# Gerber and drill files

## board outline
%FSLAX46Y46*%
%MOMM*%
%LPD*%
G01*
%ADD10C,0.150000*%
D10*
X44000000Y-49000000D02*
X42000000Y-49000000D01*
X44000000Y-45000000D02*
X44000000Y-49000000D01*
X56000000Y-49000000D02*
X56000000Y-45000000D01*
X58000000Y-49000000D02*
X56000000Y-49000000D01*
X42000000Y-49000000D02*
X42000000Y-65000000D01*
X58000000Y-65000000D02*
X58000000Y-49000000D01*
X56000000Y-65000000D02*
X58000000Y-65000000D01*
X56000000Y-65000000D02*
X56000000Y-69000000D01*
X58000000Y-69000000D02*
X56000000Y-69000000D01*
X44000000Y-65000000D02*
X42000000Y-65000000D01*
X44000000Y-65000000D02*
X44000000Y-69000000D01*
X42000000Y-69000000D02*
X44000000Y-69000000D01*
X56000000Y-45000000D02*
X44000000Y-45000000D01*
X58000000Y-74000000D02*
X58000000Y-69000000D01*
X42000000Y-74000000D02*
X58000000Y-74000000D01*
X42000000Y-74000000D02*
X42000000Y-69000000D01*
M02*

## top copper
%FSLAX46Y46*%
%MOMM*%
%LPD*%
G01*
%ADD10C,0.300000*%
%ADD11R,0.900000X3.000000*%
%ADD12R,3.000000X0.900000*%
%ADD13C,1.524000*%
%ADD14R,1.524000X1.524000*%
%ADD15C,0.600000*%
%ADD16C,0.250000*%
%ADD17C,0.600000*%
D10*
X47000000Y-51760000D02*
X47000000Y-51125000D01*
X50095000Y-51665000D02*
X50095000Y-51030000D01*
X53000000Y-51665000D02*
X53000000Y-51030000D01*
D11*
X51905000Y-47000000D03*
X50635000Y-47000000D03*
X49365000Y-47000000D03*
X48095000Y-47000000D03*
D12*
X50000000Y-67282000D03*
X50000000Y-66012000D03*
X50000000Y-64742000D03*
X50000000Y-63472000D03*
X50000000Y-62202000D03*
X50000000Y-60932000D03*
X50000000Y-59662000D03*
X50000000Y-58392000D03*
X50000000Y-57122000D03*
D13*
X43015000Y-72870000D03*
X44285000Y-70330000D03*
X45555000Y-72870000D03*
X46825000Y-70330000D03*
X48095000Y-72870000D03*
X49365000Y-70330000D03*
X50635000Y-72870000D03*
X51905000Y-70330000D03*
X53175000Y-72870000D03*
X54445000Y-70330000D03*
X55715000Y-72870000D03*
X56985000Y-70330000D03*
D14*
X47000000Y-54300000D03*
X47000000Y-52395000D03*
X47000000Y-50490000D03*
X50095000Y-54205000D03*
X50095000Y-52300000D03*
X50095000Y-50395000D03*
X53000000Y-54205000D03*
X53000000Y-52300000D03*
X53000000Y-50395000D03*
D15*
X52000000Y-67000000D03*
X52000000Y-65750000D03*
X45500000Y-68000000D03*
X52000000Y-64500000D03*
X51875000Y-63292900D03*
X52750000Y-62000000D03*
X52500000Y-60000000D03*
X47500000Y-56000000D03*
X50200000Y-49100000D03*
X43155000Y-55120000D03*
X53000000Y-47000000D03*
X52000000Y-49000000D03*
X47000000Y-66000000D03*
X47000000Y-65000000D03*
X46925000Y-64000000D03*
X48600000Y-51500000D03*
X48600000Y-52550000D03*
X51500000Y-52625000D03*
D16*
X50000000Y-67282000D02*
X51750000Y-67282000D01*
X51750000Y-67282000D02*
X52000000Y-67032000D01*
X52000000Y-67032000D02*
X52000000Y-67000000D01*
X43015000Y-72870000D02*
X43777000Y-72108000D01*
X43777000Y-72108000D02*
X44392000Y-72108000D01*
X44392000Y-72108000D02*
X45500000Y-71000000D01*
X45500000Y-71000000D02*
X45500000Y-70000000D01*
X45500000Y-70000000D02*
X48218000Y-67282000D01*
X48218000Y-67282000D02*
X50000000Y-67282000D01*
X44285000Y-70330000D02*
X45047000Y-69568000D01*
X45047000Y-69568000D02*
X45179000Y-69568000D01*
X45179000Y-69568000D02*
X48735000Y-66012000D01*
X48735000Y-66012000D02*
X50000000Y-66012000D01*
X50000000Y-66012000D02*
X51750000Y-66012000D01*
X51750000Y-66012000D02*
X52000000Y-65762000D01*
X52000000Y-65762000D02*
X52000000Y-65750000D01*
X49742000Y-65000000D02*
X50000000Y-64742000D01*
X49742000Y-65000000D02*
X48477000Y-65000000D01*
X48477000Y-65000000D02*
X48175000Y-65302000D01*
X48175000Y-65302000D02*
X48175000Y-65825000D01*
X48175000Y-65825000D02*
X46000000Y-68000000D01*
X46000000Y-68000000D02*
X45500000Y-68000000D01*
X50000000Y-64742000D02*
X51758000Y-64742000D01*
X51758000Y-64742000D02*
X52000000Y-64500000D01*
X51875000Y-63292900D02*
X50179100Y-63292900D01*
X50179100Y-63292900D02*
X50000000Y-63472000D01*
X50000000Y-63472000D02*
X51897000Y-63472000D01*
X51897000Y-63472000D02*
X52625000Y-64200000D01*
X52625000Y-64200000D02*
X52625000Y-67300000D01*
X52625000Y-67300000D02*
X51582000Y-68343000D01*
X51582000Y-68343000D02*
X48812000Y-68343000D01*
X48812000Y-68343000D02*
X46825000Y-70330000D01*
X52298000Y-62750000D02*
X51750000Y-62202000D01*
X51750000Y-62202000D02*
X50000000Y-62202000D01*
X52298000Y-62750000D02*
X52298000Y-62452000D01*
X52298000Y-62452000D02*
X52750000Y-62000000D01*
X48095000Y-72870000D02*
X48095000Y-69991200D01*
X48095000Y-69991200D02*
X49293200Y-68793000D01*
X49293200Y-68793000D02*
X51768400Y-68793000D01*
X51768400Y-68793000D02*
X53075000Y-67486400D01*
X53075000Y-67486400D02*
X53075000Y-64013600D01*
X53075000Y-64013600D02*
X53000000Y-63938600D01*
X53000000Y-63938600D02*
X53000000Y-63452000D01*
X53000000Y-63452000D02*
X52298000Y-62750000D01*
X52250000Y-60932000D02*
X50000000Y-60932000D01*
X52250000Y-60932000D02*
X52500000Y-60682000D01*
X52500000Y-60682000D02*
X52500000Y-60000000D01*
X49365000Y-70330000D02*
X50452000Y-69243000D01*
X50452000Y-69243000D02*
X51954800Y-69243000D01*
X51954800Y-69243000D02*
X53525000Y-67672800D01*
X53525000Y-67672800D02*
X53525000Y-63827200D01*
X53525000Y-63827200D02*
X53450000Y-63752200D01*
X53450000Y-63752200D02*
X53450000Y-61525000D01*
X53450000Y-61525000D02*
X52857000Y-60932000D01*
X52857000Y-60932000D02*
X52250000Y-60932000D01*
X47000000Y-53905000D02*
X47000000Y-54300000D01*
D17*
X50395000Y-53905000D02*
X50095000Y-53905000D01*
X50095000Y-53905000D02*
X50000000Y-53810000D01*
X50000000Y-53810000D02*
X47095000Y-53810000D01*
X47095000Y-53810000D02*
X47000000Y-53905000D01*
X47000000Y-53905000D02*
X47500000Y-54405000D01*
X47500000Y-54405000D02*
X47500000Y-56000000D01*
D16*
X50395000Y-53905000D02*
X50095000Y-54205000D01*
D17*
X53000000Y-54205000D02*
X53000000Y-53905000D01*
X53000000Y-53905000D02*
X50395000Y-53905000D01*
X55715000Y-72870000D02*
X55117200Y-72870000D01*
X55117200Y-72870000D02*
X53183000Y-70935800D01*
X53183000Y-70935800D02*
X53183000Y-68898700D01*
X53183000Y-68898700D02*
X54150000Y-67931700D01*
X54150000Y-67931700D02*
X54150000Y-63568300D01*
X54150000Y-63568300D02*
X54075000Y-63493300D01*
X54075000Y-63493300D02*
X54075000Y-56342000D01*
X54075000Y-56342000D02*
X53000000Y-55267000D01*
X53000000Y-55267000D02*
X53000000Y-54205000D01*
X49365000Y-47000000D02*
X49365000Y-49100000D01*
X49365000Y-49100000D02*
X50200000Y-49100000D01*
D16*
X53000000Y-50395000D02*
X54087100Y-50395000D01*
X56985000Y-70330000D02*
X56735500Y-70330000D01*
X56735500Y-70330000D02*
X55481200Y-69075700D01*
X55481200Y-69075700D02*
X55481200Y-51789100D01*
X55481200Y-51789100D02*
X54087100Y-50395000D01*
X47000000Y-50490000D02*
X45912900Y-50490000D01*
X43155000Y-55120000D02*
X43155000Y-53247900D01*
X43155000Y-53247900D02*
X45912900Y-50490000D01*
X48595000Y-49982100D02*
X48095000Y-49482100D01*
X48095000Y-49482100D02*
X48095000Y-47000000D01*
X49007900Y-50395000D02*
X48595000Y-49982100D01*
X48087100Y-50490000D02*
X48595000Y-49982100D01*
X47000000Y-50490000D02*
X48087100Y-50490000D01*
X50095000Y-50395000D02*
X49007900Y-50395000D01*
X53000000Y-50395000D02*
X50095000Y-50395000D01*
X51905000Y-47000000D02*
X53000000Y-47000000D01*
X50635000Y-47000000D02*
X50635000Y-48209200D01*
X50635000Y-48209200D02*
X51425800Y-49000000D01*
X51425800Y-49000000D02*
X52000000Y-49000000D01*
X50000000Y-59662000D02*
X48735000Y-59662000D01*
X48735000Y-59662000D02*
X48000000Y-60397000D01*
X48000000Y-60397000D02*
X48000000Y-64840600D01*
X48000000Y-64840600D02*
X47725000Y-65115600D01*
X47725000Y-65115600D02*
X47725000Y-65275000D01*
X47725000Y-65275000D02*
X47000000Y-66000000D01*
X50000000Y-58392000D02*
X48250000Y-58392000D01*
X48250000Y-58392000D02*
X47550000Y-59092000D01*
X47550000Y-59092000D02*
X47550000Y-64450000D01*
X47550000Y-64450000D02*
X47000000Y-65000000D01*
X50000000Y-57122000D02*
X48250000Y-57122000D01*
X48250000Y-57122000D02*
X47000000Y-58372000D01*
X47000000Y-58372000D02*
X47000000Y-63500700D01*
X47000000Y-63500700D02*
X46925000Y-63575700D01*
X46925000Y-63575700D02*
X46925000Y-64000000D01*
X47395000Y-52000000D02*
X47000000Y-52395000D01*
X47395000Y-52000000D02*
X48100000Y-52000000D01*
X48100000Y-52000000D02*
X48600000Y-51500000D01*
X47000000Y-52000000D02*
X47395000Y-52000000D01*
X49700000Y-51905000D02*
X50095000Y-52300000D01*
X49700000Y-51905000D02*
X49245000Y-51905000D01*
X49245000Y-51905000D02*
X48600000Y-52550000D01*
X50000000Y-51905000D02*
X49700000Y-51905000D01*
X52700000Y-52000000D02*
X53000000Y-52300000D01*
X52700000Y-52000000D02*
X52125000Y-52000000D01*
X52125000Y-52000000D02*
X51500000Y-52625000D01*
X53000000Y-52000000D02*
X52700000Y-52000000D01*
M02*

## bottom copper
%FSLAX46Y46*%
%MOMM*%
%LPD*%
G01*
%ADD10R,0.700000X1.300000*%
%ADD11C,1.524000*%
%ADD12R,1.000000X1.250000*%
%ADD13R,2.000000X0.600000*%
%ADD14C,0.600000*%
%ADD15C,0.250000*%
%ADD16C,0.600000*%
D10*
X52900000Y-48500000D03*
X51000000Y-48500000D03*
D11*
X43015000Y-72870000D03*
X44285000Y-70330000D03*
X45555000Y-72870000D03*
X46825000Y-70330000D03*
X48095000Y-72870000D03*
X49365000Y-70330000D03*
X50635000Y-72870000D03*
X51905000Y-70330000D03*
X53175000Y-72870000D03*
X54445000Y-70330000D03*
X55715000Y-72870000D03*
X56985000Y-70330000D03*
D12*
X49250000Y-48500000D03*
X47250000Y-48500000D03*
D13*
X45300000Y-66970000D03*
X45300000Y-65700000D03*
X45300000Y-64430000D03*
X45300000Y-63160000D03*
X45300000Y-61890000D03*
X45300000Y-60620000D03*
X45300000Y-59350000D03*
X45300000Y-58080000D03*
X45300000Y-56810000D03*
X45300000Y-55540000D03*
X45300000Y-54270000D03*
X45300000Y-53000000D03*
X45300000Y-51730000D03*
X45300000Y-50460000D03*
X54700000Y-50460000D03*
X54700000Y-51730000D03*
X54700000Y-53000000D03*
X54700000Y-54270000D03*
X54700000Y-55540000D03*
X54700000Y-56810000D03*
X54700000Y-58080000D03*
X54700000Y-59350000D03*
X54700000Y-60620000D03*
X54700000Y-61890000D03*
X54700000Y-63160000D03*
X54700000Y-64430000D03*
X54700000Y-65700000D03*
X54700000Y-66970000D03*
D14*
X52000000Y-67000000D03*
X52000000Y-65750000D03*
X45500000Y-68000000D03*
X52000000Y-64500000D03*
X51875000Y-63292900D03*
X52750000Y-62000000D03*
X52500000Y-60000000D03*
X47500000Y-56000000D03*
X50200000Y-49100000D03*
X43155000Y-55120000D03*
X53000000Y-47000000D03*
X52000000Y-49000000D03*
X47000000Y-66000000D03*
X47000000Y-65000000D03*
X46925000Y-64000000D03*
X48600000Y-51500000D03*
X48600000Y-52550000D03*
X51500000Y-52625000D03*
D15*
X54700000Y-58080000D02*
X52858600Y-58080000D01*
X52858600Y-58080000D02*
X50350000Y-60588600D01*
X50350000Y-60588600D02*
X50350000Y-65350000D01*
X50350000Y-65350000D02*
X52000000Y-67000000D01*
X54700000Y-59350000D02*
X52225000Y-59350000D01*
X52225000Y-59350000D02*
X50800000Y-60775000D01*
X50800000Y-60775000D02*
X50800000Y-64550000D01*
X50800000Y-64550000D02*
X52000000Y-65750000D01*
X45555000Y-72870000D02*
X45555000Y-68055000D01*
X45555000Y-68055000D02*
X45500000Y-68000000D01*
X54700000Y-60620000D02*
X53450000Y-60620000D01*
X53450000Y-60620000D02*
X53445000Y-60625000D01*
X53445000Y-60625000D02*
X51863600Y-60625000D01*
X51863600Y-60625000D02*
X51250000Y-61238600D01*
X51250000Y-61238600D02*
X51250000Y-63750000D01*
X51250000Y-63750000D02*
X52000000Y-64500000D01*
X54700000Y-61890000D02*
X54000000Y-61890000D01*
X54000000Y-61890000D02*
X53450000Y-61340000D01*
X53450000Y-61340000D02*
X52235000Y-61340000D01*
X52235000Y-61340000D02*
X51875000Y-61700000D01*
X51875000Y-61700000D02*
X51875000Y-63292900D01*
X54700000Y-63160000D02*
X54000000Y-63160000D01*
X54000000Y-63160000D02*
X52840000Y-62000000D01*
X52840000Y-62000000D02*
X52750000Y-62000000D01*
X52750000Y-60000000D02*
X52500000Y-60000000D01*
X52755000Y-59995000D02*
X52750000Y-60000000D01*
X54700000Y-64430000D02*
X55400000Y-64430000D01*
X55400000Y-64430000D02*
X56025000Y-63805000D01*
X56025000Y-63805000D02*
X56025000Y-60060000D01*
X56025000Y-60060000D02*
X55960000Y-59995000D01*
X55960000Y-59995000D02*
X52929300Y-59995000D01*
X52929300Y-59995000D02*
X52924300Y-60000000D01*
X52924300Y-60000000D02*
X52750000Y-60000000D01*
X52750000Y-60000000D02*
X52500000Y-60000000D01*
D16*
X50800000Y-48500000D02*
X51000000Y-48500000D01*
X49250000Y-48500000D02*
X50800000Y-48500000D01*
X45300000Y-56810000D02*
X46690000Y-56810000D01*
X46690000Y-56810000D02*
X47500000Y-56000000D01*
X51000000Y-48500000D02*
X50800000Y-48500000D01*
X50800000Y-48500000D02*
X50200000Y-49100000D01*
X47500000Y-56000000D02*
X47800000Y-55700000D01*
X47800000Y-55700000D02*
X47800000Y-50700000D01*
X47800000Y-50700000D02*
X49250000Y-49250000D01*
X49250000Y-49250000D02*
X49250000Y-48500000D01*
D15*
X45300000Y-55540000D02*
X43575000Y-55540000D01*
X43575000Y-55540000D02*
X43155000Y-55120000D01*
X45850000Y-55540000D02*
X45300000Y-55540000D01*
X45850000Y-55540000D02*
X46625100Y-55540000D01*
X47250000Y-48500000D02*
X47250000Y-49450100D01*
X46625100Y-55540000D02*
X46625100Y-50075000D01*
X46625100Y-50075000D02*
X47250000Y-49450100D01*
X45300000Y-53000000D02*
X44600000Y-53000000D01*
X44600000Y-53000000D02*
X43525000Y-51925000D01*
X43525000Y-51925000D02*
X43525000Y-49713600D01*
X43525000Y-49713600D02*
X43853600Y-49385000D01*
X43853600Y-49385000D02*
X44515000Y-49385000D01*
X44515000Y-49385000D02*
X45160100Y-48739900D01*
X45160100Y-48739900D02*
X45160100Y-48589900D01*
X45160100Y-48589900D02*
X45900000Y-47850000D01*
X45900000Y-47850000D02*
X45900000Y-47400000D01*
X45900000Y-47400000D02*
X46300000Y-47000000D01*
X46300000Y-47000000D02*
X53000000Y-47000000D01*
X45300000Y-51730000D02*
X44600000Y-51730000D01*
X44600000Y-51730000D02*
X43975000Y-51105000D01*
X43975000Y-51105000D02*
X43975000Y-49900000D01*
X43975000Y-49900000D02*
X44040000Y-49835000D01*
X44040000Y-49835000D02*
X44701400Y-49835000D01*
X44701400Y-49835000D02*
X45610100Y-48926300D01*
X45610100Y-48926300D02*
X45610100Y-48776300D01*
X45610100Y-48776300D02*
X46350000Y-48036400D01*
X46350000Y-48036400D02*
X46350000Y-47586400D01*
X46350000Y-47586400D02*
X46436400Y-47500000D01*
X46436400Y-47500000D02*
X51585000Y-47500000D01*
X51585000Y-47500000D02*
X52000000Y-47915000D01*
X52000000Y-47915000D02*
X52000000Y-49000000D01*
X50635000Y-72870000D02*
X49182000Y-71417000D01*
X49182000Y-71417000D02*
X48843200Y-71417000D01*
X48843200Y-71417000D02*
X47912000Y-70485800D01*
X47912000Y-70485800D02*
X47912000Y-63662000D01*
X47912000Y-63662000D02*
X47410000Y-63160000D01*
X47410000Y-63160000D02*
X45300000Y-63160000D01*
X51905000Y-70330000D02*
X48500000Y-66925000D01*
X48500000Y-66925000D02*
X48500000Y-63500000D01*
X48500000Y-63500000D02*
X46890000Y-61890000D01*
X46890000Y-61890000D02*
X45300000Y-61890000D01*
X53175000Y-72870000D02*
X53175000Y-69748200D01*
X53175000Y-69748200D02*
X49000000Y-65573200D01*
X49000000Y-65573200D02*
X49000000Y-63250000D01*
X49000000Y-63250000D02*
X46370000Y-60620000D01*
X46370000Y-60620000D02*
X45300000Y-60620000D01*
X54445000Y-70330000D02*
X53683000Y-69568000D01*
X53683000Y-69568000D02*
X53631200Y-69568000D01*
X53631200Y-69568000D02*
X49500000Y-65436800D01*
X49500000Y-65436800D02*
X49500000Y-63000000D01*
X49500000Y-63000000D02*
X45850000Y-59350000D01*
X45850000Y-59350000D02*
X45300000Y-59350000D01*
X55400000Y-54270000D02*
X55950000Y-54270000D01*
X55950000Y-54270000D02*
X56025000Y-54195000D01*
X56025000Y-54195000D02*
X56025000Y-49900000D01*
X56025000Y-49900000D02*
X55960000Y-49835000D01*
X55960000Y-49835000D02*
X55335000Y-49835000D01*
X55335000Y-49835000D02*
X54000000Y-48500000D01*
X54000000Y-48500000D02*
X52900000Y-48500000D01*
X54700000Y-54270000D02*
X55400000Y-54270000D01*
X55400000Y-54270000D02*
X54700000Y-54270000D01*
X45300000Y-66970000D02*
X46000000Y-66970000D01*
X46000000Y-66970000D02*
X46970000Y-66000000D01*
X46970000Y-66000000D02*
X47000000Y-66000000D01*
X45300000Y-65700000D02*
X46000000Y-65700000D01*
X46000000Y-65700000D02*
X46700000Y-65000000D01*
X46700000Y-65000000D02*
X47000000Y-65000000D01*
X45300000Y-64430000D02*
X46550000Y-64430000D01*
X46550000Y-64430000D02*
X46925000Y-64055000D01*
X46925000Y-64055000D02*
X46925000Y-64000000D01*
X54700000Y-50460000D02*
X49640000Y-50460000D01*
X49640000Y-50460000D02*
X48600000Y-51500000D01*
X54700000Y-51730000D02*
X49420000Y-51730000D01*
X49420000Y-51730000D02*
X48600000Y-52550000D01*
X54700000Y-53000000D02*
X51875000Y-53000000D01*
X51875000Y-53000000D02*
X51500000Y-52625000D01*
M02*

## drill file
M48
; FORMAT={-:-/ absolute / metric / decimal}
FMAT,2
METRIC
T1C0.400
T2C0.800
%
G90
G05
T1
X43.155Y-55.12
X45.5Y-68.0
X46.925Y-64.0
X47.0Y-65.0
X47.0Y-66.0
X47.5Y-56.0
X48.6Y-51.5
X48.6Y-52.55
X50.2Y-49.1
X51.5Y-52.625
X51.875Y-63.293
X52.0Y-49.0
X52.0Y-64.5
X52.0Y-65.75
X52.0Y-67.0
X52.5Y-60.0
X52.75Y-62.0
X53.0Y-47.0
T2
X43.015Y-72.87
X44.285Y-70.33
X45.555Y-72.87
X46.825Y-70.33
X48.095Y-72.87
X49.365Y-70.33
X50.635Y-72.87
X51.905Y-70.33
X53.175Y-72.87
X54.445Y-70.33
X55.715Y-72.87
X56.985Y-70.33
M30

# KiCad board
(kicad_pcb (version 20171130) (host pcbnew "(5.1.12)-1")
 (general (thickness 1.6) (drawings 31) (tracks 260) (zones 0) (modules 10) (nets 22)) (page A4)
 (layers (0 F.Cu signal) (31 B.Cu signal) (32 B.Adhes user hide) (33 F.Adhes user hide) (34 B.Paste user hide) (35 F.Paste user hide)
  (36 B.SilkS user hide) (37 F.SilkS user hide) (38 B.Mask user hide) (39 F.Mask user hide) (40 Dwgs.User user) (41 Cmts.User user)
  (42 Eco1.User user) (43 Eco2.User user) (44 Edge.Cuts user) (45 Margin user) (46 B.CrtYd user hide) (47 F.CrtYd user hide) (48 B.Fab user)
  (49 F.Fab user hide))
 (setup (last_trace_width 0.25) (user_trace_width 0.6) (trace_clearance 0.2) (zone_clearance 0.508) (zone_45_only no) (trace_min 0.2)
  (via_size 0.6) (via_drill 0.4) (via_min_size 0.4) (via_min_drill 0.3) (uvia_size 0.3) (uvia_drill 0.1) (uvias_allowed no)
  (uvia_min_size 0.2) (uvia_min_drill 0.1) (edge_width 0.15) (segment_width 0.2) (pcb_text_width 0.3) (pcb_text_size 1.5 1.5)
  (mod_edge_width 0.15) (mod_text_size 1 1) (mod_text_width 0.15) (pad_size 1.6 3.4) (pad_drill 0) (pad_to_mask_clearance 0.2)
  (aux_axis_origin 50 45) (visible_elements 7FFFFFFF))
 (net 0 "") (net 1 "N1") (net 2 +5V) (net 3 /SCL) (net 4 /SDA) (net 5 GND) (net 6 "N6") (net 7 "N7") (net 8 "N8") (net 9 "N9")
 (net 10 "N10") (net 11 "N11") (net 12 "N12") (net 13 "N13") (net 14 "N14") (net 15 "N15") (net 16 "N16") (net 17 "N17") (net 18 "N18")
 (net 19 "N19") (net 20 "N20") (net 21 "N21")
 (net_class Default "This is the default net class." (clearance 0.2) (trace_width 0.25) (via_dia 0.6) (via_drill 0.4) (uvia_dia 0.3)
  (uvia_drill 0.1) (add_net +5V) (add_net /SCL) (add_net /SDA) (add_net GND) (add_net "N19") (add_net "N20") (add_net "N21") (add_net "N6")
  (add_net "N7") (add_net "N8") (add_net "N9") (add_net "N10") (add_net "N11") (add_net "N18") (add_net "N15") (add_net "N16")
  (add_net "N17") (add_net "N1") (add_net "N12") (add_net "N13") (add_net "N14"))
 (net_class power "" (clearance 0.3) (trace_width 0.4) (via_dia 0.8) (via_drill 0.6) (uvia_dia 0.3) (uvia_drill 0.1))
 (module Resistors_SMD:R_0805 (layer B.Cu) (at 51.95 48.5 180)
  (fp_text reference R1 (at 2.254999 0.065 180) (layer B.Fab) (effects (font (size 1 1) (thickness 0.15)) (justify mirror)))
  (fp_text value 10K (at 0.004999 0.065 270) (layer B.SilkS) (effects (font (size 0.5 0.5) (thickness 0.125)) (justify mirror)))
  (pad 1 smd rect (at -0.95 0 180) (size 0.7 1.3) (layers B.Cu B.Paste B.Mask) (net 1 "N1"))
  (pad 2 smd rect (at 0.95 0 180) (size 0.7 1.3) (layers B.Cu B.Paste B.Mask) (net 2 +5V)))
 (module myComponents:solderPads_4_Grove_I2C (layer F.Cu) (at 50 47 180)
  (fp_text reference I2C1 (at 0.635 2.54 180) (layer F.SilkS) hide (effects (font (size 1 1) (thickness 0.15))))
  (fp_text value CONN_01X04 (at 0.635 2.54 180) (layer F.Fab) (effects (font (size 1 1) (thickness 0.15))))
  (pad 1 smd rect (at -1.905 0 180) (size 0.9 3) (layers F.Cu F.Paste F.Mask) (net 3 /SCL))
  (pad 2 smd rect (at -0.635 0 180) (size 0.9 3) (layers F.Cu F.Paste F.Mask) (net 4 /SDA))
  (pad 3 smd rect (at 0.635 0 180) (size 0.9 3) (layers F.Cu F.Paste F.Mask) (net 2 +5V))
  (pad 4 smd rect (at 1.905 0 180) (size 0.9 3) (layers F.Cu F.Paste F.Mask) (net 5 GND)))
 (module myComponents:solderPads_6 (layer F.Cu) (at 50 64.107 90)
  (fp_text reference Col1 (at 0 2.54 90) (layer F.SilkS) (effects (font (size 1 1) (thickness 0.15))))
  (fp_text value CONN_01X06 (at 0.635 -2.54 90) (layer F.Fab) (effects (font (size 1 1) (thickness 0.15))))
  (pad 1 smd rect (at -3.175 0 90) (size 0.9 3) (layers F.Cu F.Paste F.Mask) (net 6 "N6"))
  (pad 2 smd rect (at -1.905 0 90) (size 0.9 3) (layers F.Cu F.Paste F.Mask) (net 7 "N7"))
  (pad 3 smd rect (at -0.635 0 90) (size 0.9 3) (layers F.Cu F.Paste F.Mask) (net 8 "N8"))
  (pad 4 smd rect (at 0.635 0 90) (size 0.9 3) (layers F.Cu F.Paste F.Mask) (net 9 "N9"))
  (pad 5 smd rect (at 1.905 0 90) (size 0.9 3) (layers F.Cu F.Paste F.Mask) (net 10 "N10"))
  (pad 6 smd rect (at 3.175 0 90) (size 0.9 3) (layers F.Cu F.Paste F.Mask) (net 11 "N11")))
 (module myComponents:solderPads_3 (layer F.Cu) (at 50 58.392 90)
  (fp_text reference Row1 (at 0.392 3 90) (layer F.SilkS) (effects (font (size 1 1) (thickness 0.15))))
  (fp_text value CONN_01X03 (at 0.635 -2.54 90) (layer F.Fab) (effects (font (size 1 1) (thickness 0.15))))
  (pad 1 smd rect (at -1.27 0 90) (size 0.9 3) (layers F.Cu F.Paste F.Mask) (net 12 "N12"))
  (pad 2 smd rect (at 0 0 90) (size 0.9 3) (layers F.Cu F.Paste F.Mask) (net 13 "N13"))
  (pad 3 smd rect (at 1.27 0 90) (size 0.9 3) (layers F.Cu F.Paste F.Mask) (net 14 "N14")))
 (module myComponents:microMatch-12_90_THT (layer F.Cu) (at 50 71.6)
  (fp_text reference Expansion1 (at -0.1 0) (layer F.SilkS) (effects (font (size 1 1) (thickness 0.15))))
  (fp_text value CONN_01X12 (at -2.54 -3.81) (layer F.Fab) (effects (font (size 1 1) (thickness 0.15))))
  (pad 1 thru_hole circle (at -6.985 1.27) (size 1.524 1.524) (drill 0.8) (layers *.Cu *.Mask) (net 6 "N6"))
  (pad 2 thru_hole circle (at -5.715 -1.27) (size 1.524 1.524) (drill 0.8) (layers *.Cu *.Mask) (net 7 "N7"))
  (pad 3 thru_hole circle (at -4.445 1.27) (size 1.524 1.524) (drill 0.8) (layers *.Cu *.Mask) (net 8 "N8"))
  (pad 4 thru_hole circle (at -3.175 -1.27) (size 1.524 1.524) (drill 0.8) (layers *.Cu *.Mask) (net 9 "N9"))
  (pad 5 thru_hole circle (at -1.905 1.27) (size 1.524 1.524) (drill 0.8) (layers *.Cu *.Mask) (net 10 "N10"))
  (pad 6 thru_hole circle (at -0.635 -1.27) (size 1.524 1.524) (drill 0.8) (layers *.Cu *.Mask) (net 11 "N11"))
  (pad 7 thru_hole circle (at 0.635 1.27) (size 1.524 1.524) (drill 0.8) (layers *.Cu *.Mask) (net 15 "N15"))
  (pad 8 thru_hole circle (at 1.905 -1.27) (size 1.524 1.524) (drill 0.8) (layers *.Cu *.Mask) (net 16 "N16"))
  (pad 9 thru_hole circle (at 3.175 1.27) (size 1.524 1.524) (drill 0.8) (layers *.Cu *.Mask) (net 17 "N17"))
  (pad 10 thru_hole circle (at 4.445 -1.27) (size 1.524 1.524) (drill 0.8) (layers *.Cu *.Mask) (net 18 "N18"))
  (pad 11 thru_hole circle (at 5.715 1.27) (size 1.524 1.524) (drill 0.8) (layers *.Cu *.Mask) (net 2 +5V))
  (pad 12 thru_hole circle (at 6.985 -1.27) (size 1.524 1.524) (drill 0.8) (layers *.Cu *.Mask) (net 5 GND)))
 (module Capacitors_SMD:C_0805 (layer B.Cu) (at 48.25 48.5 180)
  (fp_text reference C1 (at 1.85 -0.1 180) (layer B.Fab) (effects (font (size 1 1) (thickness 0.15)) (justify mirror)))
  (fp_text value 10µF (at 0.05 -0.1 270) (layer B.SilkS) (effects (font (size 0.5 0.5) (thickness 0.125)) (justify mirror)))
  (pad 1 smd rect (at -1 0 180) (size 1 1.25) (layers B.Cu B.Paste B.Mask) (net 2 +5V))
  (pad 2 smd rect (at 1 0 180) (size 1 1.25) (layers B.Cu B.Paste B.Mask) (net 5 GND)))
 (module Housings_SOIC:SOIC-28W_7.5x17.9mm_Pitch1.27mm (layer B.Cu) (at 50 58.715)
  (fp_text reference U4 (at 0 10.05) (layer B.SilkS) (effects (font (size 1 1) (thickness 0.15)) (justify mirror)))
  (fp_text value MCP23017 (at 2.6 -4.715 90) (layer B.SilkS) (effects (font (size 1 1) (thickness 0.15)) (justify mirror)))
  (pad 1 smd rect (at -4.7 8.255) (size 2 0.6) (layers B.Cu B.Paste B.Mask) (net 12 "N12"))
  (pad 2 smd rect (at -4.7 6.985) (size 2 0.6) (layers B.Cu B.Paste B.Mask) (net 13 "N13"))
  (pad 3 smd rect (at -4.7 5.715) (size 2 0.6) (layers B.Cu B.Paste B.Mask) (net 14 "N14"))
  (pad 4 smd rect (at -4.7 4.445) (size 2 0.6) (layers B.Cu B.Paste B.Mask) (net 15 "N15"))
  (pad 5 smd rect (at -4.7 3.175) (size 2 0.6) (layers B.Cu B.Paste B.Mask) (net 16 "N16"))
  (pad 6 smd rect (at -4.7 1.905) (size 2 0.6) (layers B.Cu B.Paste B.Mask) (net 17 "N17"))
  (pad 7 smd rect (at -4.7 0.635) (size 2 0.6) (layers B.Cu B.Paste B.Mask) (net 18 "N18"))
  (pad 8 smd rect (at -4.7 -0.635) (size 2 0.6) (layers B.Cu B.Paste B.Mask))
  (pad 9 smd rect (at -4.7 -1.905) (size 2 0.6) (layers B.Cu B.Paste B.Mask) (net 2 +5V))
  (pad 10 smd rect (at -4.7 -3.175) (size 2 0.6) (layers B.Cu B.Paste B.Mask) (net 5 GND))
  (pad 11 smd rect (at -4.7 -4.445) (size 2 0.6) (layers B.Cu B.Paste B.Mask))
  (pad 12 smd rect (at -4.7 -5.715) (size 2 0.6) (layers B.Cu B.Paste B.Mask) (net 3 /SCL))
  (pad 13 smd rect (at -4.7 -6.985) (size 2 0.6) (layers B.Cu B.Paste B.Mask) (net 4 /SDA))
  (pad 14 smd rect (at -4.7 -8.255) (size 2 0.6) (layers B.Cu B.Paste B.Mask))
  (pad 15 smd rect (at 4.7 -8.255) (size 2 0.6) (layers B.Cu B.Paste B.Mask) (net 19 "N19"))
  (pad 16 smd rect (at 4.7 -6.985) (size 2 0.6) (layers B.Cu B.Paste B.Mask) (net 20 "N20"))
  (pad 17 smd rect (at 4.7 -5.715) (size 2 0.6) (layers B.Cu B.Paste B.Mask) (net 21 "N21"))
  (pad 18 smd rect (at 4.7 -4.445) (size 2 0.6) (layers B.Cu B.Paste B.Mask) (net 1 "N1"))
  (pad 19 smd rect (at 4.7 -3.175) (size 2 0.6) (layers B.Cu B.Paste B.Mask))
  (pad 20 smd rect (at 4.7 -1.905) (size 2 0.6) (layers B.Cu B.Paste B.Mask))
  (pad 21 smd rect (at 4.7 -0.635) (size 2 0.6) (layers B.Cu B.Paste B.Mask) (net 6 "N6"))
  (pad 22 smd rect (at 4.7 0.635) (size 2 0.6) (layers B.Cu B.Paste B.Mask) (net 7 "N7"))
  (pad 23 smd rect (at 4.7 1.905) (size 2 0.6) (layers B.Cu B.Paste B.Mask) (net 8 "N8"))
  (pad 24 smd rect (at 4.7 3.175) (size 2 0.6) (layers B.Cu B.Paste B.Mask) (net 9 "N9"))
  (pad 25 smd rect (at 4.7 4.445) (size 2 0.6) (layers B.Cu B.Paste B.Mask) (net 10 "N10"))
  (pad 26 smd rect (at 4.7 5.715) (size 2 0.6) (layers B.Cu B.Paste B.Mask) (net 11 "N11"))
  (pad 27 smd rect (at 4.7 6.985) (size 2 0.6) (layers B.Cu B.Paste B.Mask))
  (pad 28 smd rect (at 4.7 8.255) (size 2 0.6) (layers B.Cu B.Paste B.Mask)))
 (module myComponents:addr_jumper (layer F.Cu) (at 47 52.395 90)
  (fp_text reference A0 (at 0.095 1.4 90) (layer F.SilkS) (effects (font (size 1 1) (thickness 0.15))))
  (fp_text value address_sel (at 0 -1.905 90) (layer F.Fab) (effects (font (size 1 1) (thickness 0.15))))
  (fp_line (start 0.635 0) (end 1.27 0) (layer F.Cu) (width 0.3))
  (pad 1 smd rect (at -1.905 0 90) (size 1.524 1.524) (layers F.Cu F.Paste F.Mask) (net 2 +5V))
  (pad 2 smd rect (at 0 0 90) (size 1.524 1.524) (layers F.Cu F.Paste F.Mask) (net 19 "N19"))
  (pad 3 smd rect (at 1.905 0 90) (size 1.524 1.524) (layers F.Cu F.Paste F.Mask) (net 5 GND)))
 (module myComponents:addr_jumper (layer F.Cu) (at 50.095 52.3 90)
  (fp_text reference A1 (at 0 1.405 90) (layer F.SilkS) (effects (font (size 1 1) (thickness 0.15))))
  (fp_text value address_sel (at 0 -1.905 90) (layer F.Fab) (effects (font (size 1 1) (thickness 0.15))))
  (fp_line (start 0.635 0) (end 1.27 0) (layer F.Cu) (width 0.3))
  (pad 1 smd rect (at -1.905 0 90) (size 1.524 1.524) (layers F.Cu F.Paste F.Mask) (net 2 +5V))
  (pad 2 smd rect (at 0 0 90) (size 1.524 1.524) (layers F.Cu F.Paste F.Mask) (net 20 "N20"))
  (pad 3 smd rect (at 1.905 0 90) (size 1.524 1.524) (layers F.Cu F.Paste F.Mask) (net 5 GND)))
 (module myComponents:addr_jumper (layer F.Cu) (at 53 52.3 90)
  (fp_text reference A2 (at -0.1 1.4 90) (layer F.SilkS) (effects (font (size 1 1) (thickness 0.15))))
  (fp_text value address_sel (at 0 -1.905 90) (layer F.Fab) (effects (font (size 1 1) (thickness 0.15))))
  (fp_line (start 0.635 0) (end 1.27 0) (layer F.Cu) (width 0.3))
  (pad 1 smd rect (at -1.905 0 90) (size 1.524 1.524) (layers F.Cu F.Paste F.Mask) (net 2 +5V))
  (pad 2 smd rect (at 0 0 90) (size 1.524 1.524) (layers F.Cu F.Paste F.Mask) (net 21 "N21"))
  (pad 3 smd rect (at 1.905 0 90) (size 1.524 1.524) (layers F.Cu F.Paste F.Mask) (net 5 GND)))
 (gr_line (start 44 49) (end 42 49) (layer Edge.Cuts) (width 0.15))
 (gr_line (start 44 45) (end 44 49) (layer Edge.Cuts) (width 0.15))
 (gr_line (start 56 49) (end 56 45) (layer Edge.Cuts) (width 0.15))
 (gr_line (start 58 49) (end 56 49) (layer Edge.Cuts) (width 0.15))
 (gr_line (start 42 49) (end 42 65) (layer Edge.Cuts) (width 0.15))
 (gr_line (start 58 65) (end 58 49) (layer Edge.Cuts) (width 0.15))
 (gr_line (start 56 65) (end 58 65) (layer Edge.Cuts) (width 0.15))
 (gr_line (start 56 65) (end 56 69) (layer Edge.Cuts) (width 0.15))
 (gr_line (start 58 69) (end 56 69) (layer Edge.Cuts) (width 0.15))
 (gr_line (start 44 65) (end 42 65) (layer Edge.Cuts) (width 0.15))
 (gr_line (start 44 65) (end 44 69) (layer Edge.Cuts) (width 0.15))
 (gr_line (start 42 69) (end 44 69) (layer Edge.Cuts) (width 0.15))
 (gr_line (start 56 45) (end 44 45) (layer Edge.Cuts) (width 0.15))
 (gr_line (start 58 74) (end 58 69) (layer Edge.Cuts) (width 0.15))
 (gr_line (start 42 74) (end 58 74) (layer Edge.Cuts) (width 0.15))
 (gr_line (start 42 74) (end 42 69) (layer Edge.Cuts) (width 0.15))
 (segment (start 50 67.282) (end 51.75 67.282) (width 0.25) (layer F.Cu) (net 6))
 (segment (start 51.75 67.282) (end 52 67.032) (width 0.25) (layer F.Cu) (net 6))
 (segment (start 52 67.032) (end 52 67) (width 0.25) (layer F.Cu) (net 6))
 (segment (start 54.7 58.08) (end 52.8586 58.08) (width 0.25) (layer B.Cu) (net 6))
 (segment (start 52.8586 58.08) (end 50.35 60.5886) (width 0.25) (layer B.Cu) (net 6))
 (segment (start 50.35 60.5886) (end 50.35 65.35) (width 0.25) (layer B.Cu) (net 6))
 (segment (start 50.35 65.35) (end 52 67) (width 0.25) (layer B.Cu) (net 6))
 (segment (start 43.015 72.87) (end 43.777 72.108) (width 0.25) (layer F.Cu) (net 6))
 (segment (start 43.777 72.108) (end 44.392 72.108) (width 0.25) (layer F.Cu) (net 6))
 (segment (start 44.392 72.108) (end 45.5 71) (width 0.25) (layer F.Cu) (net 6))
 (segment (start 45.5 71) (end 45.5 70) (width 0.25) (layer F.Cu) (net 6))
 (segment (start 45.5 70) (end 48.218 67.282) (width 0.25) (layer F.Cu) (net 6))
 (segment (start 48.218 67.282) (end 50 67.282) (width 0.25) (layer F.Cu) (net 6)) (via (at 52 67) (size 0.6) (layers F.Cu B.Cu) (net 6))
 (segment (start 44.285 70.33) (end 45.047 69.568) (width 0.25) (layer F.Cu) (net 7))
 (segment (start 45.047 69.568) (end 45.179 69.568) (width 0.25) (layer F.Cu) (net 7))
 (segment (start 45.179 69.568) (end 48.735 66.012) (width 0.25) (layer F.Cu) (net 7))
 (segment (start 48.735 66.012) (end 50 66.012) (width 0.25) (layer F.Cu) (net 7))
 (segment (start 54.7 59.35) (end 52.225 59.35) (width 0.25) (layer B.Cu) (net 7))
 (segment (start 52.225 59.35) (end 50.8 60.775) (width 0.25) (layer B.Cu) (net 7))
 (segment (start 50.8 60.775) (end 50.8 64.55) (width 0.25) (layer B.Cu) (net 7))
 (segment (start 50.8 64.55) (end 52 65.75) (width 0.25) (layer B.Cu) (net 7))
 (segment (start 50 66.012) (end 51.75 66.012) (width 0.25) (layer F.Cu) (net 7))
 (segment (start 51.75 66.012) (end 52 65.762) (width 0.25) (layer F.Cu) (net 7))
 (segment (start 52 65.762) (end 52 65.75) (width 0.25) (layer F.Cu) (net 7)) (via (at 52 65.75) (size 0.6) (layers F.Cu B.Cu) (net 7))
 (segment (start 49.742 65) (end 50 64.742) (width 0.25) (layer F.Cu) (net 8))
 (segment (start 49.742 65) (end 48.477 65) (width 0.25) (layer F.Cu) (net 8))
 (segment (start 48.477 65) (end 48.175 65.302) (width 0.25) (layer F.Cu) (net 8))
 (segment (start 48.175 65.302) (end 48.175 65.825) (width 0.25) (layer F.Cu) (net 8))
 (segment (start 48.175 65.825) (end 46 68) (width 0.25) (layer F.Cu) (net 8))
 (segment (start 46 68) (end 45.5 68) (width 0.25) (layer F.Cu) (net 8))
 (segment (start 45.555 72.87) (end 45.555 68.055) (width 0.25) (layer B.Cu) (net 8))
 (segment (start 45.555 68.055) (end 45.5 68) (width 0.25) (layer B.Cu) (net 8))
 (segment (start 54.7 60.62) (end 53.45 60.62) (width 0.25) (layer B.Cu) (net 8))
 (segment (start 53.45 60.62) (end 53.445 60.625) (width 0.25) (layer B.Cu) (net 8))
 (segment (start 53.445 60.625) (end 51.8636 60.625) (width 0.25) (layer B.Cu) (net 8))
 (segment (start 51.8636 60.625) (end 51.25 61.2386) (width 0.25) (layer B.Cu) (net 8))
 (segment (start 51.25 61.2386) (end 51.25 63.75) (width 0.25) (layer B.Cu) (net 8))
 (segment (start 51.25 63.75) (end 52 64.5) (width 0.25) (layer B.Cu) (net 8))
 (segment (start 50 64.742) (end 51.758 64.742) (width 0.25) (layer F.Cu) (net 8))
 (segment (start 51.758 64.742) (end 52 64.5) (width 0.25) (layer F.Cu) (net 8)) (via (at 45.5 68) (size 0.6) (layers F.Cu B.Cu) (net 8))
 (via (at 52 64.5) (size 0.6) (layers F.Cu B.Cu) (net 8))
 (segment (start 51.875 63.2929) (end 50.1791 63.2929) (width 0.25) (layer F.Cu) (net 9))
 (segment (start 50.1791 63.2929) (end 50 63.472) (width 0.25) (layer F.Cu) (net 9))
 (segment (start 54.7 61.89) (end 54 61.89) (width 0.25) (layer B.Cu) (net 9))
 (segment (start 54 61.89) (end 53.45 61.34) (width 0.25) (layer B.Cu) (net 9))
 (segment (start 53.45 61.34) (end 52.235 61.34) (width 0.25) (layer B.Cu) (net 9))
 (segment (start 52.235 61.34) (end 51.875 61.7) (width 0.25) (layer B.Cu) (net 9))
 (segment (start 51.875 61.7) (end 51.875 63.2929) (width 0.25) (layer B.Cu) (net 9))
 (segment (start 50 63.472) (end 51.897 63.472) (width 0.25) (layer F.Cu) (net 9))
 (segment (start 51.897 63.472) (end 52.625 64.2) (width 0.25) (layer F.Cu) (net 9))
 (segment (start 52.625 64.2) (end 52.625 67.3) (width 0.25) (layer F.Cu) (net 9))
 (segment (start 52.625 67.3) (end 51.582 68.343) (width 0.25) (layer F.Cu) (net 9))
 (segment (start 51.582 68.343) (end 48.812 68.343) (width 0.25) (layer F.Cu) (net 9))
 (segment (start 48.812 68.343) (end 46.825 70.33) (width 0.25) (layer F.Cu) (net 9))
 (via (at 51.875 63.2929) (size 0.6) (layers F.Cu B.Cu) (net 9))
 (segment (start 52.298 62.75) (end 51.75 62.202) (width 0.25) (layer F.Cu) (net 10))
 (segment (start 51.75 62.202) (end 50 62.202) (width 0.25) (layer F.Cu) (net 10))
 (segment (start 54.7 63.16) (end 54 63.16) (width 0.25) (layer B.Cu) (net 10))
 (segment (start 54 63.16) (end 52.84 62) (width 0.25) (layer B.Cu) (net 10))
 (segment (start 52.84 62) (end 52.75 62) (width 0.25) (layer B.Cu) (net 10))
 (segment (start 52.298 62.75) (end 52.298 62.452) (width 0.25) (layer F.Cu) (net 10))
 (segment (start 52.298 62.452) (end 52.75 62) (width 0.25) (layer F.Cu) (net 10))
 (segment (start 48.095 72.87) (end 48.095 69.9912) (width 0.25) (layer F.Cu) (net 10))
 (segment (start 48.095 69.9912) (end 49.2932 68.793) (width 0.25) (layer F.Cu) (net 10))
 (segment (start 49.2932 68.793) (end 51.7684 68.793) (width 0.25) (layer F.Cu) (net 10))
 (segment (start 51.7684 68.793) (end 53.075 67.4864) (width 0.25) (layer F.Cu) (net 10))
 (segment (start 53.075 67.4864) (end 53.075 64.0136) (width 0.25) (layer F.Cu) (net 10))
 (segment (start 53.075 64.0136) (end 53 63.9386) (width 0.25) (layer F.Cu) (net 10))
 (segment (start 53 63.9386) (end 53 63.452) (width 0.25) (layer F.Cu) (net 10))
 (segment (start 53 63.452) (end 52.298 62.75) (width 0.25) (layer F.Cu) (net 10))
 (via (at 52.75 62) (size 0.6) (layers F.Cu B.Cu) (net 10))
 (segment (start 52.75 60) (end 52.5 60) (width 0.25) (layer B.Cu) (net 11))
 (segment (start 52.25 60.932) (end 50 60.932) (width 0.25) (layer F.Cu) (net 11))
 (segment (start 52.25 60.932) (end 52.5 60.682) (width 0.25) (layer F.Cu) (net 11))
 (segment (start 52.5 60.682) (end 52.5 60) (width 0.25) (layer F.Cu) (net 11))
 (segment (start 52.755 59.995) (end 52.75 60) (width 0.25) (layer B.Cu) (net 11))
 (segment (start 54.7 64.43) (end 55.4 64.43) (width 0.25) (layer B.Cu) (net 11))
 (segment (start 55.4 64.43) (end 56.025 63.805) (width 0.25) (layer B.Cu) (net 11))
 (segment (start 56.025 63.805) (end 56.025 60.06) (width 0.25) (layer B.Cu) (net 11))
 (segment (start 56.025 60.06) (end 55.96 59.995) (width 0.25) (layer B.Cu) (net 11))
 (segment (start 55.96 59.995) (end 52.9293 59.995) (width 0.25) (layer B.Cu) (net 11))
 (segment (start 52.9293 59.995) (end 52.9243 60) (width 0.25) (layer B.Cu) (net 11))
 (segment (start 52.9243 60) (end 52.75 60) (width 0.25) (layer B.Cu) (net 11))
 (segment (start 52.75 60) (end 52.5 60) (width 0.25) (layer B.Cu) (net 11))
 (segment (start 49.365 70.33) (end 50.452 69.243) (width 0.25) (layer F.Cu) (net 11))
 (segment (start 50.452 69.243) (end 51.9548 69.243) (width 0.25) (layer F.Cu) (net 11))
 (segment (start 51.9548 69.243) (end 53.525 67.6728) (width 0.25) (layer F.Cu) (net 11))
 (segment (start 53.525 67.6728) (end 53.525 63.8272) (width 0.25) (layer F.Cu) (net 11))
 (segment (start 53.525 63.8272) (end 53.45 63.7522) (width 0.25) (layer F.Cu) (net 11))
 (segment (start 53.45 63.7522) (end 53.45 61.525) (width 0.25) (layer F.Cu) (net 11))
 (segment (start 53.45 61.525) (end 52.857 60.932) (width 0.25) (layer F.Cu) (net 11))
 (segment (start 52.857 60.932) (end 52.25 60.932) (width 0.25) (layer F.Cu) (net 11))
 (via (at 52.5 60) (size 0.6) (layers F.Cu B.Cu) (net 11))
 (segment (start 47 53.905) (end 47 54.3) (width 0.25) (layer F.Cu) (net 2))
 (segment (start 50.395 53.905) (end 50.095 53.905) (width 0.6) (layer F.Cu) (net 2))
 (segment (start 50.095 53.905) (end 50 53.81) (width 0.6) (layer F.Cu) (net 2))
 (segment (start 50 53.81) (end 47.095 53.81) (width 0.6) (layer F.Cu) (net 2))
 (segment (start 47.095 53.81) (end 47 53.905) (width 0.6) (layer F.Cu) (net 2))
 (segment (start 47 53.905) (end 47.5 54.405) (width 0.6) (layer F.Cu) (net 2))
 (segment (start 47.5 54.405) (end 47.5 56) (width 0.6) (layer F.Cu) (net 2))
 (segment (start 50.395 53.905) (end 50.095 54.205) (width 0.25) (layer F.Cu) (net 2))
 (segment (start 53 54.205) (end 53 53.905) (width 0.6) (layer F.Cu) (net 2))
 (segment (start 53 53.905) (end 50.395 53.905) (width 0.6) (layer F.Cu) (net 2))
 (segment (start 50.8 48.5) (end 51 48.5) (width 0.6) (layer B.Cu) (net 2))
 (segment (start 49.25 48.5) (end 50.8 48.5) (width 0.6) (layer B.Cu) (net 2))
 (segment (start 55.715 72.87) (end 55.1172 72.87) (width 0.6) (layer F.Cu) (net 2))
 (segment (start 55.1172 72.87) (end 53.183 70.9358) (width 0.6) (layer F.Cu) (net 2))
 (segment (start 53.183 70.9358) (end 53.183 68.8987) (width 0.6) (layer F.Cu) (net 2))
 (segment (start 53.183 68.8987) (end 54.15 67.9317) (width 0.6) (layer F.Cu) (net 2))
 (segment (start 54.15 67.9317) (end 54.15 63.5683) (width 0.6) (layer F.Cu) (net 2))
 (segment (start 54.15 63.5683) (end 54.075 63.4933) (width 0.6) (layer F.Cu) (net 2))
 (segment (start 54.075 63.4933) (end 54.075 56.342) (width 0.6) (layer F.Cu) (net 2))
 (segment (start 54.075 56.342) (end 53 55.267) (width 0.6) (layer F.Cu) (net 2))
 (segment (start 53 55.267) (end 53 54.205) (width 0.6) (layer F.Cu) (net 2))
 (segment (start 45.3 56.81) (end 46.69 56.81) (width 0.6) (layer B.Cu) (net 2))
 (segment (start 46.69 56.81) (end 47.5 56) (width 0.6) (layer B.Cu) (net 2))
 (segment (start 51 48.5) (end 50.8 48.5) (width 0.6) (layer B.Cu) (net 2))
 (segment (start 50.8 48.5) (end 50.2 49.1) (width 0.6) (layer B.Cu) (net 2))
 (segment (start 49.365 47) (end 49.365 49.1) (width 0.6) (layer F.Cu) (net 2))
 (segment (start 49.365 49.1) (end 50.2 49.1) (width 0.6) (layer F.Cu) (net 2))
 (segment (start 47.5 56) (end 47.8 55.7) (width 0.6) (layer B.Cu) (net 2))
 (segment (start 47.8 55.7) (end 47.8 50.7) (width 0.6) (layer B.Cu) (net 2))
 (segment (start 47.8 50.7) (end 49.25 49.25) (width 0.6) (layer B.Cu) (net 2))
 (segment (start 49.25 49.25) (end 49.25 48.5) (width 0.6) (layer B.Cu) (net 2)) (via (at 47.5 56) (size 0.6) (layers F.Cu B.Cu) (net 2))
 (via (at 50.2 49.1) (size 0.6) (layers F.Cu B.Cu) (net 2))
 (segment (start 53 50.395) (end 54.0871 50.395) (width 0.25) (layer F.Cu) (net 5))
 (segment (start 56.985 70.33) (end 56.7355 70.33) (width 0.25) (layer F.Cu) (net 5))
 (segment (start 56.7355 70.33) (end 55.4812 69.0757) (width 0.25) (layer F.Cu) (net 5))
 (segment (start 55.4812 69.0757) (end 55.4812 51.7891) (width 0.25) (layer F.Cu) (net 5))
 (segment (start 55.4812 51.7891) (end 54.0871 50.395) (width 0.25) (layer F.Cu) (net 5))
 (segment (start 47 50.49) (end 45.9129 50.49) (width 0.25) (layer F.Cu) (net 5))
 (segment (start 43.155 55.12) (end 43.155 53.2479) (width 0.25) (layer F.Cu) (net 5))
 (segment (start 43.155 53.2479) (end 45.9129 50.49) (width 0.25) (layer F.Cu) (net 5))
 (segment (start 45.3 55.54) (end 43.575 55.54) (width 0.25) (layer B.Cu) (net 5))
 (segment (start 43.575 55.54) (end 43.155 55.12) (width 0.25) (layer B.Cu) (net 5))
 (segment (start 45.85 55.54) (end 45.3 55.54) (width 0.25) (layer B.Cu) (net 5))
 (segment (start 45.85 55.54) (end 46.6251 55.54) (width 0.25) (layer B.Cu) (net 5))
 (segment (start 47.25 48.5) (end 47.25 49.4501) (width 0.25) (layer B.Cu) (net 5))
 (segment (start 46.6251 55.54) (end 46.6251 50.075) (width 0.25) (layer B.Cu) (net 5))
 (segment (start 46.6251 50.075) (end 47.25 49.4501) (width 0.25) (layer B.Cu) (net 5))
 (segment (start 48.595 49.9821) (end 48.095 49.4821) (width 0.25) (layer F.Cu) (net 5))
 (segment (start 48.095 49.4821) (end 48.095 47) (width 0.25) (layer F.Cu) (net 5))
 (segment (start 49.0079 50.395) (end 48.595 49.9821) (width 0.25) (layer F.Cu) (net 5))
 (segment (start 48.0871 50.49) (end 48.595 49.9821) (width 0.25) (layer F.Cu) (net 5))
 (segment (start 47 50.49) (end 48.0871 50.49) (width 0.25) (layer F.Cu) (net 5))
 (segment (start 50.095 50.395) (end 49.0079 50.395) (width 0.25) (layer F.Cu) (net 5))
 (segment (start 53 50.395) (end 50.095 50.395) (width 0.25) (layer F.Cu) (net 5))
 (via (at 43.155 55.12) (size 0.6) (layers F.Cu B.Cu) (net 5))
 (segment (start 51.905 47) (end 53 47) (width 0.25) (layer F.Cu) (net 3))
 (segment (start 45.3 53) (end 44.6 53) (width 0.25) (layer B.Cu) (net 3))
 (segment (start 44.6 53) (end 43.525 51.925) (width 0.25) (layer B.Cu) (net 3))
 (segment (start 43.525 51.925) (end 43.525 49.7136) (width 0.25) (layer B.Cu) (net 3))
 (segment (start 43.525 49.7136) (end 43.8536 49.385) (width 0.25) (layer B.Cu) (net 3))
 (segment (start 43.8536 49.385) (end 44.515 49.385) (width 0.25) (layer B.Cu) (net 3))
 (segment (start 44.515 49.385) (end 45.1601 48.7399) (width 0.25) (layer B.Cu) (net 3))
 (segment (start 45.1601 48.7399) (end 45.1601 48.5899) (width 0.25) (layer B.Cu) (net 3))
 (segment (start 45.1601 48.5899) (end 45.9 47.85) (width 0.25) (layer B.Cu) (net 3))
 (segment (start 45.9 47.85) (end 45.9 47.4) (width 0.25) (layer B.Cu) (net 3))
 (segment (start 45.9 47.4) (end 46.3 47) (width 0.25) (layer B.Cu) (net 3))
 (segment (start 46.3 47) (end 53 47) (width 0.25) (layer B.Cu) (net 3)) (via (at 53 47) (size 0.6) (layers F.Cu B.Cu) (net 3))
 (segment (start 50.635 47) (end 50.635 48.2092) (width 0.25) (layer F.Cu) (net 4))
 (segment (start 50.635 48.2092) (end 51.4258 49) (width 0.25) (layer F.Cu) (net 4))
 (segment (start 51.4258 49) (end 52 49) (width 0.25) (layer F.Cu) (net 4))
 (segment (start 45.3 51.73) (end 44.6 51.73) (width 0.25) (layer B.Cu) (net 4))
 (segment (start 44.6 51.73) (end 43.975 51.105) (width 0.25) (layer B.Cu) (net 4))
 (segment (start 43.975 51.105) (end 43.975 49.9) (width 0.25) (layer B.Cu) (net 4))
 (segment (start 43.975 49.9) (end 44.04 49.835) (width 0.25) (layer B.Cu) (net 4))
 (segment (start 44.04 49.835) (end 44.7014 49.835) (width 0.25) (layer B.Cu) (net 4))
 (segment (start 44.7014 49.835) (end 45.6101 48.9263) (width 0.25) (layer B.Cu) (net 4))
 (segment (start 45.6101 48.9263) (end 45.6101 48.7763) (width 0.25) (layer B.Cu) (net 4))
 (segment (start 45.6101 48.7763) (end 46.35 48.0364) (width 0.25) (layer B.Cu) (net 4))
 (segment (start 46.35 48.0364) (end 46.35 47.5864) (width 0.25) (layer B.Cu) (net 4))
 (segment (start 46.35 47.5864) (end 46.4364 47.5) (width 0.25) (layer B.Cu) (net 4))
 (segment (start 46.4364 47.5) (end 51.585 47.5) (width 0.25) (layer B.Cu) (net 4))
 (segment (start 51.585 47.5) (end 52 47.915) (width 0.25) (layer B.Cu) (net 4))
 (segment (start 52 47.915) (end 52 49) (width 0.25) (layer B.Cu) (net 4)) (via (at 52 49) (size 0.6) (layers F.Cu B.Cu) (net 4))
 (segment (start 50.635 72.87) (end 49.182 71.417) (width 0.25) (layer B.Cu) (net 15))
 (segment (start 49.182 71.417) (end 48.8432 71.417) (width 0.25) (layer B.Cu) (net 15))
 (segment (start 48.8432 71.417) (end 47.912 70.4858) (width 0.25) (layer B.Cu) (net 15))
 (segment (start 47.912 70.4858) (end 47.912 63.662) (width 0.25) (layer B.Cu) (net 15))
 (segment (start 47.912 63.662) (end 47.41 63.16) (width 0.25) (layer B.Cu) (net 15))
 (segment (start 47.41 63.16) (end 45.3 63.16) (width 0.25) (layer B.Cu) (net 15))
 (segment (start 51.905 70.33) (end 48.5 66.925) (width 0.25) (layer B.Cu) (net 16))
 (segment (start 48.5 66.925) (end 48.5 63.5) (width 0.25) (layer B.Cu) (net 16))
 (segment (start 48.5 63.5) (end 46.89 61.89) (width 0.25) (layer B.Cu) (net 16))
 (segment (start 46.89 61.89) (end 45.3 61.89) (width 0.25) (layer B.Cu) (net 16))
 (segment (start 53.175 72.87) (end 53.175 69.7482) (width 0.25) (layer B.Cu) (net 17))
 (segment (start 53.175 69.7482) (end 49 65.5732) (width 0.25) (layer B.Cu) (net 17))
 (segment (start 49 65.5732) (end 49 63.25) (width 0.25) (layer B.Cu) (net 17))
 (segment (start 49 63.25) (end 46.37 60.62) (width 0.25) (layer B.Cu) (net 17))
 (segment (start 46.37 60.62) (end 45.3 60.62) (width 0.25) (layer B.Cu) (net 17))
 (segment (start 54.445 70.33) (end 53.683 69.568) (width 0.25) (layer B.Cu) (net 18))
 (segment (start 53.683 69.568) (end 53.6312 69.568) (width 0.25) (layer B.Cu) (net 18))
 (segment (start 53.6312 69.568) (end 49.5 65.4368) (width 0.25) (layer B.Cu) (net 18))
 (segment (start 49.5 65.4368) (end 49.5 63) (width 0.25) (layer B.Cu) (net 18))
 (segment (start 49.5 63) (end 45.85 59.35) (width 0.25) (layer B.Cu) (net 18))
 (segment (start 45.85 59.35) (end 45.3 59.35) (width 0.25) (layer B.Cu) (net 18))
 (segment (start 55.4 54.27) (end 55.95 54.27) (width 0.25) (layer B.Cu) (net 1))
 (segment (start 55.95 54.27) (end 56.025 54.195) (width 0.25) (layer B.Cu) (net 1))
 (segment (start 56.025 54.195) (end 56.025 49.9) (width 0.25) (layer B.Cu) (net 1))
 (segment (start 56.025 49.9) (end 55.96 49.835) (width 0.25) (layer B.Cu) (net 1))
 (segment (start 55.96 49.835) (end 55.335 49.835) (width 0.25) (layer B.Cu) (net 1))
 (segment (start 55.335 49.835) (end 54 48.5) (width 0.25) (layer B.Cu) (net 1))
 (segment (start 54 48.5) (end 52.9 48.5) (width 0.25) (layer B.Cu) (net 1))
 (segment (start 54.7 54.27) (end 55.4 54.27) (width 0.25) (layer B.Cu) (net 1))
 (segment (start 55.4 54.27) (end 54.7 54.27) (width 0.25) (layer B.Cu) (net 1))
 (segment (start 45.3 66.97) (end 46 66.97) (width 0.25) (layer B.Cu) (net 12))
 (segment (start 46 66.97) (end 46.97 66) (width 0.25) (layer B.Cu) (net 12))
 (segment (start 46.97 66) (end 47 66) (width 0.25) (layer B.Cu) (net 12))
 (segment (start 50 59.662) (end 48.735 59.662) (width 0.25) (layer F.Cu) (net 12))
 (segment (start 48.735 59.662) (end 48 60.397) (width 0.25) (layer F.Cu) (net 12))
 (segment (start 48 60.397) (end 48 64.8406) (width 0.25) (layer F.Cu) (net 12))
 (segment (start 48 64.8406) (end 47.725 65.1156) (width 0.25) (layer F.Cu) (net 12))
 (segment (start 47.725 65.1156) (end 47.725 65.275) (width 0.25) (layer F.Cu) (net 12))
 (segment (start 47.725 65.275) (end 47 66) (width 0.25) (layer F.Cu) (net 12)) (via (at 47 66) (size 0.6) (layers F.Cu B.Cu) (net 12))
 (segment (start 45.3 65.7) (end 46 65.7) (width 0.25) (layer B.Cu) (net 13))
 (segment (start 46 65.7) (end 46.7 65) (width 0.25) (layer B.Cu) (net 13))
 (segment (start 46.7 65) (end 47 65) (width 0.25) (layer B.Cu) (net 13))
 (segment (start 50 58.392) (end 48.25 58.392) (width 0.25) (layer F.Cu) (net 13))
 (segment (start 48.25 58.392) (end 47.55 59.092) (width 0.25) (layer F.Cu) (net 13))
 (segment (start 47.55 59.092) (end 47.55 64.45) (width 0.25) (layer F.Cu) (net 13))
 (segment (start 47.55 64.45) (end 47 65) (width 0.25) (layer F.Cu) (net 13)) (via (at 47 65) (size 0.6) (layers F.Cu B.Cu) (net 13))
 (segment (start 45.3 64.43) (end 46.55 64.43) (width 0.25) (layer B.Cu) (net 14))
 (segment (start 46.55 64.43) (end 46.925 64.055) (width 0.25) (layer B.Cu) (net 14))
 (segment (start 46.925 64.055) (end 46.925 64) (width 0.25) (layer B.Cu) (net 14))
 (segment (start 50 57.122) (end 48.25 57.122) (width 0.25) (layer F.Cu) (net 14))
 (segment (start 48.25 57.122) (end 47 58.372) (width 0.25) (layer F.Cu) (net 14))
 (segment (start 47 58.372) (end 47 63.5007) (width 0.25) (layer F.Cu) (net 14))
 (segment (start 47 63.5007) (end 46.925 63.5757) (width 0.25) (layer F.Cu) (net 14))
 (segment (start 46.925 63.5757) (end 46.925 64) (width 0.25) (layer F.Cu) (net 14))
 (via (at 46.925 64) (size 0.6) (layers F.Cu B.Cu) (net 14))
 (segment (start 47.395 52) (end 47 52.395) (width 0.25) (layer F.Cu) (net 19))
 (segment (start 47.395 52) (end 48.1 52) (width 0.25) (layer F.Cu) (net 19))
 (segment (start 48.1 52) (end 48.6 51.5) (width 0.25) (layer F.Cu) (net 19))
 (segment (start 47 52) (end 47.395 52) (width 0.25) (layer F.Cu) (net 19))
 (segment (start 54.7 50.46) (end 49.64 50.46) (width 0.25) (layer B.Cu) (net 19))
 (segment (start 49.64 50.46) (end 48.6 51.5) (width 0.25) (layer B.Cu) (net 19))
 (via (at 48.6 51.5) (size 0.6) (layers F.Cu B.Cu) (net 19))
 (segment (start 49.7 51.905) (end 50.095 52.3) (width 0.25) (layer F.Cu) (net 20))
 (segment (start 49.7 51.905) (end 49.245 51.905) (width 0.25) (layer F.Cu) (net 20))
 (segment (start 49.245 51.905) (end 48.6 52.55) (width 0.25) (layer F.Cu) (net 20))
 (segment (start 50 51.905) (end 49.7 51.905) (width 0.25) (layer F.Cu) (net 20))
 (segment (start 54.7 51.73) (end 49.42 51.73) (width 0.25) (layer B.Cu) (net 20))
 (segment (start 49.42 51.73) (end 48.6 52.55) (width 0.25) (layer B.Cu) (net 20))
 (via (at 48.6 52.55) (size 0.6) (layers F.Cu B.Cu) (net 20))
 (segment (start 52.7 52) (end 53 52.3) (width 0.25) (layer F.Cu) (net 21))
 (segment (start 52.7 52) (end 52.125 52) (width 0.25) (layer F.Cu) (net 21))
 (segment (start 52.125 52) (end 51.5 52.625) (width 0.25) (layer F.Cu) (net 21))
 (segment (start 53 52) (end 52.7 52) (width 0.25) (layer F.Cu) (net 21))
 (segment (start 54.7 53) (end 51.875 53) (width 0.25) (layer B.Cu) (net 21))
 (segment (start 51.875 53) (end 51.5 52.625) (width 0.25) (layer B.Cu) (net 21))
 (via (at 51.5 52.625) (size 0.6) (layers F.Cu B.Cu) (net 21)))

